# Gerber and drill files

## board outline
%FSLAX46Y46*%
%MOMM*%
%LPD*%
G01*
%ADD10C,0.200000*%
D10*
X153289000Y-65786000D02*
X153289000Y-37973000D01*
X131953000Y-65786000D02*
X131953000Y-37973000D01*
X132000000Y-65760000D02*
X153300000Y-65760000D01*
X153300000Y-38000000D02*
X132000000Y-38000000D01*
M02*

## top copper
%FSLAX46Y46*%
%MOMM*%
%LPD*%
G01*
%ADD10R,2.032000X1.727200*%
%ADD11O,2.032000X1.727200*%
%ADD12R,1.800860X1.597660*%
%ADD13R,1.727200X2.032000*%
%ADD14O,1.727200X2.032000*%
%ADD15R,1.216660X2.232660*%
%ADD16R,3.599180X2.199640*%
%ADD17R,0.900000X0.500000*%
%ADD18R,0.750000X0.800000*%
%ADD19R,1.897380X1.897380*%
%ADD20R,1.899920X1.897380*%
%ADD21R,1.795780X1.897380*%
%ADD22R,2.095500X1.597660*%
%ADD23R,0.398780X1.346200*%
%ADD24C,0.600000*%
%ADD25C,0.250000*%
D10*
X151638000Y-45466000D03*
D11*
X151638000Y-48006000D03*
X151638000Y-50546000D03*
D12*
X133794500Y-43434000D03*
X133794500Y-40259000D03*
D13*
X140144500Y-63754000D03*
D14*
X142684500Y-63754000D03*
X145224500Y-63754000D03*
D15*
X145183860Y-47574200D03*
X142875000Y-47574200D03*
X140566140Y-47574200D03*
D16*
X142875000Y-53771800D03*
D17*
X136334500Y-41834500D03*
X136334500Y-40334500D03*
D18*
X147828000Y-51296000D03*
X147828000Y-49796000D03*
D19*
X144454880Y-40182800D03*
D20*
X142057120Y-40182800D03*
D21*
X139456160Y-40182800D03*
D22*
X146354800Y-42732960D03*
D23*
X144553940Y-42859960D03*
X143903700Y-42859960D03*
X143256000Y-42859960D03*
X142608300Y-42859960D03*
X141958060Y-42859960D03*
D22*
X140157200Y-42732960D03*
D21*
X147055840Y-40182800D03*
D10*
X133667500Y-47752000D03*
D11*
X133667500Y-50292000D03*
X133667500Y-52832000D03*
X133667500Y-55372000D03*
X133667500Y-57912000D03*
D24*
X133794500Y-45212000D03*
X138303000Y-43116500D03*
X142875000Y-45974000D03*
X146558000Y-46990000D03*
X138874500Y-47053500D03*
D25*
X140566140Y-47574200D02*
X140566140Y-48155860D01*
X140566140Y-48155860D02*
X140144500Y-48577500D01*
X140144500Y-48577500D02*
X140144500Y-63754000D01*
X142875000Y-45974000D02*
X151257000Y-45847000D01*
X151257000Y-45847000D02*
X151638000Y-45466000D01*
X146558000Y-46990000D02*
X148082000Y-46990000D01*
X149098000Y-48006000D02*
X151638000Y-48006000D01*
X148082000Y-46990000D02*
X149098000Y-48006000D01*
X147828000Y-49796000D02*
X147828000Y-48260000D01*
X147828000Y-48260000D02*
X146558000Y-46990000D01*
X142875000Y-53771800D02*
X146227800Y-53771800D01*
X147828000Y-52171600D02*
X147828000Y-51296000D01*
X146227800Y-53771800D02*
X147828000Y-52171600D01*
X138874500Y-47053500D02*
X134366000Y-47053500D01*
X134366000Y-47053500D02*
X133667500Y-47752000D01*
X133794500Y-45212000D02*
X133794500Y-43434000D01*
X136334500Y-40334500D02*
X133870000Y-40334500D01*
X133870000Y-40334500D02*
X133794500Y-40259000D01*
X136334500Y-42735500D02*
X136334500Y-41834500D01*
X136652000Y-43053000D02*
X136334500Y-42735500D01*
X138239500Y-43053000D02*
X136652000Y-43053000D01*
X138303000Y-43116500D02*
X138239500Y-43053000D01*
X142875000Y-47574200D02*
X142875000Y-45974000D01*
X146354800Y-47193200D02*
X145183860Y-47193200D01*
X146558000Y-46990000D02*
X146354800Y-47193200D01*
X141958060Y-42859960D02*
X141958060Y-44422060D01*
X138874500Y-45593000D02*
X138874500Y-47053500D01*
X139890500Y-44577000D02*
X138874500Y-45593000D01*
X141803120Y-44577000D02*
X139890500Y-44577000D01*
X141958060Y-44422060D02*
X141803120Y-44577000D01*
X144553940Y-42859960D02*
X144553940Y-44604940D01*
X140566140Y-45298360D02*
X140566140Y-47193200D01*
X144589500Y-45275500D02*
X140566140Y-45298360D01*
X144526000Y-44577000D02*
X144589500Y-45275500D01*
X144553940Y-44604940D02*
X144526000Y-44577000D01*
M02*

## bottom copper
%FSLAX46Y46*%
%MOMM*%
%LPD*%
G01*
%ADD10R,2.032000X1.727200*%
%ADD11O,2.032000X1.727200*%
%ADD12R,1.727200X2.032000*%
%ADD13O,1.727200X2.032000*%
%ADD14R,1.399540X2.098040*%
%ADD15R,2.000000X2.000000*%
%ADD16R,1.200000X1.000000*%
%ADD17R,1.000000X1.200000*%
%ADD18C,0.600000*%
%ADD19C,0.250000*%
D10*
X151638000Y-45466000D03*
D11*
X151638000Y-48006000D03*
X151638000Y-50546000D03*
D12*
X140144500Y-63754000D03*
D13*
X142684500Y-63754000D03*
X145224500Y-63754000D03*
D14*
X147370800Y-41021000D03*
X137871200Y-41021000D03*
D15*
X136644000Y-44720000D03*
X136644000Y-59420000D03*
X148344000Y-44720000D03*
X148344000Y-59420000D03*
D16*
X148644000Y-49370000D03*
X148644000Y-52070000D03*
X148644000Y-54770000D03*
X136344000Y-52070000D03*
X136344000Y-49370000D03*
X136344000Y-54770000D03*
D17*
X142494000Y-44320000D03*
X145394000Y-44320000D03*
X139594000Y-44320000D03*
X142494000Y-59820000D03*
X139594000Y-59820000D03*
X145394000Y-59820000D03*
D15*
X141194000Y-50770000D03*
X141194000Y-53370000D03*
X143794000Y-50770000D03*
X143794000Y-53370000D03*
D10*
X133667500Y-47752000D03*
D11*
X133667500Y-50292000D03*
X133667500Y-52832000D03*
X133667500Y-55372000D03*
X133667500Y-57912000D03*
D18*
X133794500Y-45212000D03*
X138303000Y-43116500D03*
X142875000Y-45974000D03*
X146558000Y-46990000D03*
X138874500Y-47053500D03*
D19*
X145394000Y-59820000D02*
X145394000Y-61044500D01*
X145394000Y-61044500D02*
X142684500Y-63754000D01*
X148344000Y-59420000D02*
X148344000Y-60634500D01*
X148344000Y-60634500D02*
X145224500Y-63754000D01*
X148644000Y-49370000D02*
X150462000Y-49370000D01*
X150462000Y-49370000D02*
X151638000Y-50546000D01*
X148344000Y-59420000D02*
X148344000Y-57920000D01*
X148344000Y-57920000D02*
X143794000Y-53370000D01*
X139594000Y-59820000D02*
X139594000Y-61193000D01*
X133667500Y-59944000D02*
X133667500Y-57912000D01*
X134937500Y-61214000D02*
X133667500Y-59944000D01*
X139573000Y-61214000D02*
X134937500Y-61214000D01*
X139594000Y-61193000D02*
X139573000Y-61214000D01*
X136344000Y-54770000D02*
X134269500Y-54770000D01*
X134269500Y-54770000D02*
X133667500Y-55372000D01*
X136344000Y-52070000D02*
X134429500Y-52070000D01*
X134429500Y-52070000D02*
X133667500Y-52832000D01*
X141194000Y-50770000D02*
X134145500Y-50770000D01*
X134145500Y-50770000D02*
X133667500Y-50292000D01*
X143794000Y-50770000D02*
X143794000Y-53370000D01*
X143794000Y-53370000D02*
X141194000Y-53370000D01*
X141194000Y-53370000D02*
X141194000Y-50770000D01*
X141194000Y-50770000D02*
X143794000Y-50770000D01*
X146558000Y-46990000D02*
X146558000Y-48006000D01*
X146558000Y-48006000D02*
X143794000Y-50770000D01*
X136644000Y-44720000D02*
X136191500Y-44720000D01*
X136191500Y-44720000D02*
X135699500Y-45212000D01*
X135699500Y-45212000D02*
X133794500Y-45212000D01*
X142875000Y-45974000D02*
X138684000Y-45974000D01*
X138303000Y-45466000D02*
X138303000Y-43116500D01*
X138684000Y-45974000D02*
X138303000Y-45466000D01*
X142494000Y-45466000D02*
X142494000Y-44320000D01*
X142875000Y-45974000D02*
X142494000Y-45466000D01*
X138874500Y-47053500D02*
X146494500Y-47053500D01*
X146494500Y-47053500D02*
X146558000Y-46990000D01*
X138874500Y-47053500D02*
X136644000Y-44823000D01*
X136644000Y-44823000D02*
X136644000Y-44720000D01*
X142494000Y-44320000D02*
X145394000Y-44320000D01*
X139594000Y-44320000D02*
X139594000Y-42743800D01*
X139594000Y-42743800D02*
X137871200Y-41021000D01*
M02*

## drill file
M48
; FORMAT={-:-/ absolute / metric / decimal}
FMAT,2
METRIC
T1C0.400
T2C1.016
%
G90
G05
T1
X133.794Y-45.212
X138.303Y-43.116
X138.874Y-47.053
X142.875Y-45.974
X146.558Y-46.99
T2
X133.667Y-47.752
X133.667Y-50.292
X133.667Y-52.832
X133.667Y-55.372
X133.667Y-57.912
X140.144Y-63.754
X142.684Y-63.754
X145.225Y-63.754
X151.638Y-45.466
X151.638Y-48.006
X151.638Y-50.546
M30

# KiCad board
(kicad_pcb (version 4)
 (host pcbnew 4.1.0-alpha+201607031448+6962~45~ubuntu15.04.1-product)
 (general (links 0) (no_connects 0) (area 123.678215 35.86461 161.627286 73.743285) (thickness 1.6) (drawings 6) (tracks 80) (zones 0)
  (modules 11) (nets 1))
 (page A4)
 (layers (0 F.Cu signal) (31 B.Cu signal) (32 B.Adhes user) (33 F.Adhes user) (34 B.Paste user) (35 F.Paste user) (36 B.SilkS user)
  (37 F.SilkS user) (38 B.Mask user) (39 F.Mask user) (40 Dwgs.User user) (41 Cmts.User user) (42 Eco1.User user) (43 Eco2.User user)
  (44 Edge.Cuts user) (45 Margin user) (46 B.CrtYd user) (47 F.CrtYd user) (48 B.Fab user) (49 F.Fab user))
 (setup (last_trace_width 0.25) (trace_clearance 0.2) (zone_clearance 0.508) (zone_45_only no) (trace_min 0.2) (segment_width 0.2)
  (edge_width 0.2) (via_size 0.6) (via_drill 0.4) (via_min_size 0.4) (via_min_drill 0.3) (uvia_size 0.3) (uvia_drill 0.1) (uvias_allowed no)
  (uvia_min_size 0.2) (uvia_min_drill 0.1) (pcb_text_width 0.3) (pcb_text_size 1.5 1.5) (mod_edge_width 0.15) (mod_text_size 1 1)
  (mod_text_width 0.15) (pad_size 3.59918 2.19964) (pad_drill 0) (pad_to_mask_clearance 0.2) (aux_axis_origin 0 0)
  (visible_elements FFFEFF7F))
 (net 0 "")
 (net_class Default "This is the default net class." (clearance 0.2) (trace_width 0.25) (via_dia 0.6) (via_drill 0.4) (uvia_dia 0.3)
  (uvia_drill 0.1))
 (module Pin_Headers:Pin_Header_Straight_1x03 (layer F.Cu) (at 151.638 45.466)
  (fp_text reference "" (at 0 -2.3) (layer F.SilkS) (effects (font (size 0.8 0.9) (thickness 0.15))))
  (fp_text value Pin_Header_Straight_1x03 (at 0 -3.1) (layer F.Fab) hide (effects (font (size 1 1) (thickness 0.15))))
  (pad 1 thru_hole rect (at 0 0) (size 2.032 1.7272) (drill 1.016) (layers *.Cu *.Mask F.SilkS))
  (pad 2 thru_hole oval (at 0 2.54) (size 2.032 1.7272) (drill 1.016) (layers *.Cu *.Mask F.SilkS))
  (pad 3 thru_hole oval (at 0 5.08) (size 2.032 1.7272) (drill 1.016) (layers *.Cu *.Mask F.SilkS)))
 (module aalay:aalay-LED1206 (layer F.Cu) (at 133.7945 41.8465 90)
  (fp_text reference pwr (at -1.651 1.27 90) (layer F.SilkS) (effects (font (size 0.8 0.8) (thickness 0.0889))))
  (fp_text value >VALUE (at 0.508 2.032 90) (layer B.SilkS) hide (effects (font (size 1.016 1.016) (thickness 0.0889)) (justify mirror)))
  (pad A smd rect (at -1.5875 0 90) (size 1.59766 1.80086) (layers F.Cu F.Paste F.Mask))
  (pad K smd rect (at 1.5875 0 90) (size 1.59766 1.80086) (layers F.Cu F.Paste F.Mask)))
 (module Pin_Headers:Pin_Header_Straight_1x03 (layer F.Cu) (at 140.1445 63.754 90)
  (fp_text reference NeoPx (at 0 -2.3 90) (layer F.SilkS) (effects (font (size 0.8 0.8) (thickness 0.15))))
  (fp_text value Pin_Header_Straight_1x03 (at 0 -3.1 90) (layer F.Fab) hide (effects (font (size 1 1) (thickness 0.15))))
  (pad 1 thru_hole rect (at 0 0 90) (size 2.032 1.7272) (drill 1.016) (layers *.Cu *.Mask F.SilkS))
  (pad 2 thru_hole oval (at 0 2.54 90) (size 2.032 1.7272) (drill 1.016) (layers *.Cu *.Mask F.SilkS))
  (pad 3 thru_hole oval (at 0 5.08 90) (size 2.032 1.7272) (drill 1.016) (layers *.Cu *.Mask F.SilkS)))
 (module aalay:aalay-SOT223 (layer F.Cu) (at 142.875 50.673 180)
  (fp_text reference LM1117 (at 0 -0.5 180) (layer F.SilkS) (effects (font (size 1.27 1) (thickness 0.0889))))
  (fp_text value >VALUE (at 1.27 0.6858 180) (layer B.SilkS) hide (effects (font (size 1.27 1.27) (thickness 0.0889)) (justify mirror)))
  (pad GND smd rect (at -2.30886 3.0988 180) (size 1.21666 2.23266) (layers F.Cu F.Paste F.Mask))
  (pad OUT smd rect (at 0 3.0988 180) (size 1.21666 2.23266) (layers F.Cu F.Paste F.Mask))
  (pad IN smd rect (at 2.30886 3.0988 180) (size 1.21666 2.23266) (layers F.Cu F.Paste F.Mask))
  (pad OUT smd rect (at 0 -3.0988 180) (size 3.59918 2.19964) (layers F.Cu F.Paste F.Mask)))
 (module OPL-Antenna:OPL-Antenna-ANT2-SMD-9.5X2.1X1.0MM (layer B.Cu) (at 142.621 41.021 180)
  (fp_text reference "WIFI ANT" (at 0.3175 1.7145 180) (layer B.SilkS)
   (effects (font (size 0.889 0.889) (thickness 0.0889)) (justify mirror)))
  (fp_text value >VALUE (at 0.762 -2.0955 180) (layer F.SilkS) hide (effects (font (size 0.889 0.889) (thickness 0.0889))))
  (pad 1 smd rect (at -4.7498 0 180) (size 1.39954 2.09804) (layers B.Cu B.Paste B.Mask))
  (pad 2 smd rect (at 4.7498 0 180) (size 1.39954 2.09804) (layers B.Cu B.Paste B.Mask)))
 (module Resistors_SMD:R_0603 (layer F.Cu) (at 136.3345 41.0845 90)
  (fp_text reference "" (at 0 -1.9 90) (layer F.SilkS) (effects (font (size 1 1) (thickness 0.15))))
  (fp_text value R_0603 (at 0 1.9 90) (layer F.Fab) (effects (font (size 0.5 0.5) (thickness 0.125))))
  (pad 1 smd rect (at -0.75 0 90) (size 0.5 0.9) (layers F.Cu F.Paste F.Mask))
  (pad 2 smd rect (at 0.75 0 90) (size 0.5 0.9) (layers F.Cu F.Paste F.Mask)))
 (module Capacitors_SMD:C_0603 (layer F.Cu) (at 147.828 50.546 90)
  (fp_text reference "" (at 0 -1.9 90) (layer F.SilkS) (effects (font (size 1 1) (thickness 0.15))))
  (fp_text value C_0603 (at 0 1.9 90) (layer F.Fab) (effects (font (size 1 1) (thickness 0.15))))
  (pad 1 smd rect (at -0.75 0 90) (size 0.8 0.75) (layers F.Cu F.Paste F.Mask))
  (pad 2 smd rect (at 0.75 0 90) (size 0.8 0.75) (layers F.Cu F.Paste F.Mask)))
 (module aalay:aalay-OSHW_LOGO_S (layer F.Cu) (at 150.622 39.878)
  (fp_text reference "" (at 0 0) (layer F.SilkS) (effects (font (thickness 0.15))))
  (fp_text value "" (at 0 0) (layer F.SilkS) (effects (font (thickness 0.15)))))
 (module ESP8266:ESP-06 (layer B.Cu) (at 142.494 52.07 270)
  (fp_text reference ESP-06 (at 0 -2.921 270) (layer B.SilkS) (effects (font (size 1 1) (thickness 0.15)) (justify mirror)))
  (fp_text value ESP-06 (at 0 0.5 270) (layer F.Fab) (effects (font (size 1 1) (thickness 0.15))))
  (pad GND smd rect (at -7.35 5.85 270) (size 2 2) (layers B.Cu B.Paste B.Mask))
  (pad GP5 smd rect (at 7.35 5.85 270) (size 2 2) (layers B.Cu B.Paste B.Mask))
  (pad GP16 smd rect (at -7.35 -5.85 270) (size 2 2) (layers B.Cu B.Paste B.Mask))
  (pad GP15 smd rect (at 7.35 -5.85 270) (size 2 2) (layers B.Cu B.Paste B.Mask))
  (pad GP14 smd rect (at -2.7 -6.15 270) (size 1 1.2) (layers B.Cu B.Paste B.Mask))
  (pad GP12 smd rect (at 0 -6.15 270) (size 1 1.2) (layers B.Cu B.Paste B.Mask))
  (pad GP13 smd rect (at 2.7 -6.15 270) (size 1 1.2) (layers B.Cu B.Paste B.Mask))
  (pad TX smd rect (at 0 6.15 270) (size 1 1.2) (layers B.Cu B.Paste B.Mask))
  (pad RST smd rect (at -2.7 6.15 270) (size 1 1.2) (layers B.Cu B.Paste B.Mask))
  (pad RX smd rect (at 2.7 6.15 270) (size 1 1.2) (layers B.Cu B.Paste B.Mask))
  (pad 3.3 smd rect (at -7.75 0 270) (size 1.2 1) (layers B.Cu B.Paste B.Mask))
  (pad CHPD smd rect (at -7.75 -2.9 270) (size 1.2 1) (layers B.Cu B.Paste B.Mask))
  (pad ANT smd rect (at -7.75 2.9 270) (size 1.2 1) (layers B.Cu B.Paste B.Mask))
  (pad GP2 smd rect (at 7.75 0 270) (size 1.2 1) (layers B.Cu B.Paste B.Mask))
  (pad GP0 smd rect (at 7.75 2.9 270) (size 1.2 1) (layers B.Cu B.Paste B.Mask))
  (pad GP4 smd rect (at 7.75 -2.9 270) (size 1.2 1) (layers B.Cu B.Paste B.Mask))
  (pad GND smd rect (at -1.3 1.3 270) (size 2 2) (layers B.Cu B.Paste B.Mask))
  (pad GND smd rect (at 1.3 1.3 270) (size 2 2) (layers B.Cu B.Paste B.Mask))
  (pad GND smd rect (at -1.3 -1.3 270) (size 2 2) (layers B.Cu B.Paste B.Mask))
  (pad GND smd rect (at 1.3 -1.3 270) (size 2 2) (layers B.Cu B.Paste B.Mask)))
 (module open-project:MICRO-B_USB (layer F.Cu) (at 143.256 38.735 180)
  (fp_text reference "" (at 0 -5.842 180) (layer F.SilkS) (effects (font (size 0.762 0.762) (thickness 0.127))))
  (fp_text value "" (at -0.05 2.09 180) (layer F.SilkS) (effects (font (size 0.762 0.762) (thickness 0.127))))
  (pad "" smd rect (at -1.19888 -1.4478 180) (size 1.89738 1.89738) (layers F.Cu F.Paste F.Mask))
  (pad "" smd rect (at 1.19888 -1.4478 180) (size 1.89992 1.89738) (layers F.Cu F.Paste F.Mask))
  (pad "" smd rect (at 3.79984 -1.4478 180) (size 1.79578 1.89738) (layers F.Cu F.Paste F.Mask))
  (pad "" smd rect (at -3.0988 -3.99796 180) (size 2.0955 1.59766) (layers F.Cu F.Paste F.Mask))
  (pad 1 smd rect (at -1.29794 -4.12496 180) (size 0.39878 1.3462) (layers F.Cu F.Paste F.Mask) (clearance 0.2032))
  (pad 2 smd rect (at -0.6477 -4.12496 180) (size 0.39878 1.3462) (layers F.Cu F.Paste F.Mask) (clearance 0.2032))
  (pad 3 smd rect (at 0 -4.12496 180) (size 0.39878 1.3462) (layers F.Cu F.Paste F.Mask) (clearance 0.2032))
  (pad 4 smd rect (at 0.6477 -4.12496 180) (size 0.39878 1.3462) (layers F.Cu F.Paste F.Mask) (clearance 0.2032))
  (pad 5 smd rect (at 1.29794 -4.12496 180) (size 0.39878 1.3462) (layers F.Cu F.Paste F.Mask) (clearance 0.2032))
  (pad "" smd rect (at 3.0988 -3.99796 180) (size 2.0955 1.59766) (layers F.Cu F.Paste F.Mask))
  (pad "" smd rect (at -3.79984 -1.4478 180) (size 1.79578 1.89738) (layers F.Cu F.Paste F.Mask)))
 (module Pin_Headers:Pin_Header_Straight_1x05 (layer F.Cu) (at 133.6675 47.752)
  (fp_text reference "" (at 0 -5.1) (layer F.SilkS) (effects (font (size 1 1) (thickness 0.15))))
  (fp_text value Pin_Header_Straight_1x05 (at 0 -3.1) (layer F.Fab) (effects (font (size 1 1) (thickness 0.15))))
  (pad 1 thru_hole rect (at 0 0) (size 2.032 1.7272) (drill 1.016) (layers *.Cu *.Mask F.SilkS))
  (pad 2 thru_hole oval (at 0 2.54) (size 2.032 1.7272) (drill 1.016) (layers *.Cu *.Mask F.SilkS))
  (pad 3 thru_hole oval (at 0 5.08) (size 2.032 1.7272) (drill 1.016) (layers *.Cu *.Mask F.SilkS))
  (pad 4 thru_hole oval (at 0 7.62) (size 2.032 1.7272) (drill 1.016) (layers *.Cu *.Mask F.SilkS))
  (pad 5 thru_hole oval (at 0 10.16) (size 2.032 1.7272) (drill 1.016) (layers *.Cu *.Mask F.SilkS)))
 (gr_line (start 153.289 65.786) (end 153.289 37.973) (angle 90) (layer Edge.Cuts) (width 0.2))
 (gr_line (start 131.953 65.786) (end 131.953 37.973) (angle 90) (layer Edge.Cuts) (width 0.2))
 (gr_line (start 132 65.76) (end 153.3 65.76) (angle 90) (layer Edge.Cuts) (width 0.2))
 (gr_line (start 153.3 38) (end 132 38) (angle 90) (layer Edge.Cuts) (width 0.2))
 (segment (start 140.56614 47.5742) (end 140.56614 48.15586) (width 0.25) (layer F.Cu) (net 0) (status C00000))
 (segment (start 140.56614 48.15586) (end 140.1445 48.5775) (width 0.25) (layer F.Cu) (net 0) (status C00000))
 (segment (start 140.1445 48.5775) (end 140.1445 63.754) (width 0.25) (layer F.Cu) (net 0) (status C00000))
 (segment (start 145.394 59.82) (end 145.394 61.0445) (width 0.25) (layer B.Cu) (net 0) (status 400000))
 (segment (start 145.394 61.0445) (end 142.6845 63.754) (width 0.25) (layer B.Cu) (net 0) (status 800000))
 (segment (start 148.344 59.42) (end 148.344 60.6345) (width 0.25) (layer B.Cu) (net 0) (status 400000))
 (segment (start 148.344 60.6345) (end 145.2245 63.754) (width 0.25) (layer B.Cu) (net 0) (status 800000))
 (segment (start 148.644 49.37) (end 150.462 49.37) (width 0.25) (layer B.Cu) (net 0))
 (segment (start 150.462 49.37) (end 151.638 50.546) (width 0.25) (layer B.Cu) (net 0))
 (segment (start 142.875 45.974) (end 151.257 45.847) (width 0.25) (layer F.Cu) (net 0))
 (segment (start 151.257 45.847) (end 151.638 45.466) (width 0.25) (layer F.Cu) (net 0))
 (segment (start 146.558 46.99) (end 148.082 46.99) (width 0.25) (layer F.Cu) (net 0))
 (segment (start 149.098 48.006) (end 151.638 48.006) (width 0.25) (layer F.Cu) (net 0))
 (segment (start 148.082 46.99) (end 149.098 48.006) (width 0.25) (layer F.Cu) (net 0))
 (segment (start 147.828 49.796) (end 147.828 48.26) (width 0.25) (layer F.Cu) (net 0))
 (segment (start 147.828 48.26) (end 146.558 46.99) (width 0.25) (layer F.Cu) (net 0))
 (segment (start 142.875 53.7718) (end 146.2278 53.7718) (width 0.25) (layer F.Cu) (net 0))
 (segment (start 147.828 52.1716) (end 147.828 51.296) (width 0.25) (layer F.Cu) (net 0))
 (segment (start 146.2278 53.7718) (end 147.828 52.1716) (width 0.25) (layer F.Cu) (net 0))
 (segment (start 148.344 59.42) (end 148.344 57.92) (width 0.25) (layer B.Cu) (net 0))
 (segment (start 148.344 57.92) (end 143.794 53.37) (width 0.25) (layer B.Cu) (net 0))
 (segment (start 139.594 59.82) (end 139.594 61.193) (width 0.25) (layer B.Cu) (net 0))
 (segment (start 133.6675 59.944) (end 133.6675 57.912) (width 0.25) (layer B.Cu) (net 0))
 (segment (start 134.9375 61.214) (end 133.6675 59.944) (width 0.25) (layer B.Cu) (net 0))
 (segment (start 139.573 61.214) (end 134.9375 61.214) (width 0.25) (layer B.Cu) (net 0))
 (segment (start 139.594 61.193) (end 139.573 61.214) (width 0.25) (layer B.Cu) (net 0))
 (segment (start 136.344 54.77) (end 134.2695 54.77) (width 0.25) (layer B.Cu) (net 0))
 (segment (start 134.2695 54.77) (end 133.6675 55.372) (width 0.25) (layer B.Cu) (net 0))
 (segment (start 136.344 52.07) (end 134.4295 52.07) (width 0.25) (layer B.Cu) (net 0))
 (segment (start 134.4295 52.07) (end 133.6675 52.832) (width 0.25) (layer B.Cu) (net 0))
 (segment (start 141.194 50.77) (end 134.1455 50.77) (width 0.25) (layer B.Cu) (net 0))
 (segment (start 134.1455 50.77) (end 133.6675 50.292) (width 0.25) (layer B.Cu) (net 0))
 (segment (start 138.8745 47.0535) (end 134.366 47.0535) (width 0.25) (layer F.Cu) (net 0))
 (segment (start 134.366 47.0535) (end 133.6675 47.752) (width 0.25) (layer F.Cu) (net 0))
 (segment (start 143.794 50.77) (end 143.794 53.37) (width 0.25) (layer B.Cu) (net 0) (status 30))
 (segment (start 143.794 53.37) (end 141.194 53.37) (width 0.25) (layer B.Cu) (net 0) (status 30))
 (segment (start 141.194 53.37) (end 141.194 50.77) (width 0.25) (layer B.Cu) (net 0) (status 30))
 (segment (start 141.194 50.77) (end 143.794 50.77) (width 0.25) (layer B.Cu) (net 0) (status 30))
 (segment (start 146.558 46.99) (end 146.558 48.006) (width 0.25) (layer B.Cu) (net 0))
 (segment (start 146.558 48.006) (end 143.794 50.77) (width 0.25) (layer B.Cu) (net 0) (status 20))
 (segment (start 136.644 44.72) (end 136.1915 44.72) (width 0.25) (layer B.Cu) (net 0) (status 30))
 (segment (start 136.1915 44.72) (end 135.6995 45.212) (width 0.25) (layer B.Cu) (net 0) (status 30))
 (segment (start 135.6995 45.212) (end 133.7945 45.212) (width 0.25) (layer B.Cu) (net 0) (status 10))
 (via (at 133.7945 45.212) (size 0.6) (drill 0.4) (layers F.Cu B.Cu) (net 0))
 (segment (start 133.7945 45.212) (end 133.7945 43.434) (width 0.25) (layer F.Cu) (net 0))
 (segment (start 136.3345 40.3345) (end 133.87 40.3345) (width 0.25) (layer F.Cu) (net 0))
 (segment (start 133.87 40.3345) (end 133.7945 40.259) (width 0.25) (layer F.Cu) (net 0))
 (segment (start 142.875 45.974) (end 138.684 45.974) (width 0.25) (layer B.Cu) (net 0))
 (segment (start 136.3345 42.7355) (end 136.3345 41.8345) (width 0.25) (layer F.Cu) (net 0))
 (segment (start 136.652 43.053) (end 136.3345 42.7355) (width 0.25) (layer F.Cu) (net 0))
 (segment (start 138.2395 43.053) (end 136.652 43.053) (width 0.25) (layer F.Cu) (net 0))
 (segment (start 138.303 43.1165) (end 138.2395 43.053) (width 0.25) (layer F.Cu) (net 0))
 (via (at 138.303 43.1165) (size 0.6) (drill 0.4) (layers F.Cu B.Cu) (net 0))
 (segment (start 138.303 45.466) (end 138.303 43.1165) (width 0.25) (layer B.Cu) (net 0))
 (segment (start 138.684 45.974) (end 138.303 45.466) (width 0.25) (layer B.Cu) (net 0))
 (segment (start 142.875 47.5742) (end 142.875 45.974) (width 0.25) (layer F.Cu) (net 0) (status 400010))
 (segment (start 142.494 45.466) (end 142.494 44.32) (width 0.25) (layer B.Cu) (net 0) (status 20))
 (segment (start 142.875 45.974) (end 142.494 45.466) (width 0.25) (layer B.Cu) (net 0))
 (via (at 142.875 45.974) (size 0.6) (drill 0.4) (layers F.Cu B.Cu) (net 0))
 (segment (start 138.8745 47.0535) (end 146.4945 47.0535) (width 0.25) (layer B.Cu) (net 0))
 (segment (start 146.3548 47.1932) (end 145.18386 47.1932) (width 0.25) (layer F.Cu) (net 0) (status 20))
 (segment (start 146.558 46.99) (end 146.3548 47.1932) (width 0.25) (layer F.Cu) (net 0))
 (via (at 146.558 46.99) (size 0.6) (drill 0.4) (layers F.Cu B.Cu) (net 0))
 (segment (start 146.4945 47.0535) (end 146.558 46.99) (width 0.25) (layer B.Cu) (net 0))
 (segment (start 141.95806 42.85996) (end 141.95806 44.42206) (width 0.25) (layer F.Cu) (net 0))
 (segment (start 138.8745 47.0535) (end 136.644 44.823) (width 0.25) (layer B.Cu) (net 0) (status 20))
 (via (at 138.8745 47.0535) (size 0.6) (drill 0.4) (layers F.Cu B.Cu) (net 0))
 (segment (start 138.8745 45.593) (end 138.8745 47.0535) (width 0.25) (layer F.Cu) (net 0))
 (segment (start 139.8905 44.577) (end 138.8745 45.593) (width 0.25) (layer F.Cu) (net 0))
 (segment (start 141.80312 44.577) (end 139.8905 44.577) (width 0.25) (layer F.Cu) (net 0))
 (segment (start 141.95806 44.42206) (end 141.80312 44.577) (width 0.25) (layer F.Cu) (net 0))
 (segment (start 136.644 44.823) (end 136.644 44.72) (width 0.25) (layer B.Cu) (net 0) (status 30))
 (segment (start 144.55394 42.85996) (end 144.55394 44.60494) (width 0.25) (layer F.Cu) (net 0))
 (segment (start 140.56614 45.29836) (end 140.56614 47.1932) (width 0.25) (layer F.Cu) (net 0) (status 20))
 (segment (start 144.5895 45.2755) (end 140.56614 45.29836) (width 0.25) (layer F.Cu) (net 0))
 (segment (start 144.526 44.577) (end 144.5895 45.2755) (width 0.25) (layer F.Cu) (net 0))
 (segment (start 144.55394 44.60494) (end 144.526 44.577) (width 0.25) (layer F.Cu) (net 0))
 (segment (start 142.494 44.32) (end 145.394 44.32) (width 0.25) (layer B.Cu) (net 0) (status 30))
 (segment (start 139.594 44.32) (end 139.594 42.7438) (width 0.25) (layer B.Cu) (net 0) (status 10))
 (segment (start 139.594 42.7438) (end 137.8712 41.021) (width 0.25) (layer B.Cu) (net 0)))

